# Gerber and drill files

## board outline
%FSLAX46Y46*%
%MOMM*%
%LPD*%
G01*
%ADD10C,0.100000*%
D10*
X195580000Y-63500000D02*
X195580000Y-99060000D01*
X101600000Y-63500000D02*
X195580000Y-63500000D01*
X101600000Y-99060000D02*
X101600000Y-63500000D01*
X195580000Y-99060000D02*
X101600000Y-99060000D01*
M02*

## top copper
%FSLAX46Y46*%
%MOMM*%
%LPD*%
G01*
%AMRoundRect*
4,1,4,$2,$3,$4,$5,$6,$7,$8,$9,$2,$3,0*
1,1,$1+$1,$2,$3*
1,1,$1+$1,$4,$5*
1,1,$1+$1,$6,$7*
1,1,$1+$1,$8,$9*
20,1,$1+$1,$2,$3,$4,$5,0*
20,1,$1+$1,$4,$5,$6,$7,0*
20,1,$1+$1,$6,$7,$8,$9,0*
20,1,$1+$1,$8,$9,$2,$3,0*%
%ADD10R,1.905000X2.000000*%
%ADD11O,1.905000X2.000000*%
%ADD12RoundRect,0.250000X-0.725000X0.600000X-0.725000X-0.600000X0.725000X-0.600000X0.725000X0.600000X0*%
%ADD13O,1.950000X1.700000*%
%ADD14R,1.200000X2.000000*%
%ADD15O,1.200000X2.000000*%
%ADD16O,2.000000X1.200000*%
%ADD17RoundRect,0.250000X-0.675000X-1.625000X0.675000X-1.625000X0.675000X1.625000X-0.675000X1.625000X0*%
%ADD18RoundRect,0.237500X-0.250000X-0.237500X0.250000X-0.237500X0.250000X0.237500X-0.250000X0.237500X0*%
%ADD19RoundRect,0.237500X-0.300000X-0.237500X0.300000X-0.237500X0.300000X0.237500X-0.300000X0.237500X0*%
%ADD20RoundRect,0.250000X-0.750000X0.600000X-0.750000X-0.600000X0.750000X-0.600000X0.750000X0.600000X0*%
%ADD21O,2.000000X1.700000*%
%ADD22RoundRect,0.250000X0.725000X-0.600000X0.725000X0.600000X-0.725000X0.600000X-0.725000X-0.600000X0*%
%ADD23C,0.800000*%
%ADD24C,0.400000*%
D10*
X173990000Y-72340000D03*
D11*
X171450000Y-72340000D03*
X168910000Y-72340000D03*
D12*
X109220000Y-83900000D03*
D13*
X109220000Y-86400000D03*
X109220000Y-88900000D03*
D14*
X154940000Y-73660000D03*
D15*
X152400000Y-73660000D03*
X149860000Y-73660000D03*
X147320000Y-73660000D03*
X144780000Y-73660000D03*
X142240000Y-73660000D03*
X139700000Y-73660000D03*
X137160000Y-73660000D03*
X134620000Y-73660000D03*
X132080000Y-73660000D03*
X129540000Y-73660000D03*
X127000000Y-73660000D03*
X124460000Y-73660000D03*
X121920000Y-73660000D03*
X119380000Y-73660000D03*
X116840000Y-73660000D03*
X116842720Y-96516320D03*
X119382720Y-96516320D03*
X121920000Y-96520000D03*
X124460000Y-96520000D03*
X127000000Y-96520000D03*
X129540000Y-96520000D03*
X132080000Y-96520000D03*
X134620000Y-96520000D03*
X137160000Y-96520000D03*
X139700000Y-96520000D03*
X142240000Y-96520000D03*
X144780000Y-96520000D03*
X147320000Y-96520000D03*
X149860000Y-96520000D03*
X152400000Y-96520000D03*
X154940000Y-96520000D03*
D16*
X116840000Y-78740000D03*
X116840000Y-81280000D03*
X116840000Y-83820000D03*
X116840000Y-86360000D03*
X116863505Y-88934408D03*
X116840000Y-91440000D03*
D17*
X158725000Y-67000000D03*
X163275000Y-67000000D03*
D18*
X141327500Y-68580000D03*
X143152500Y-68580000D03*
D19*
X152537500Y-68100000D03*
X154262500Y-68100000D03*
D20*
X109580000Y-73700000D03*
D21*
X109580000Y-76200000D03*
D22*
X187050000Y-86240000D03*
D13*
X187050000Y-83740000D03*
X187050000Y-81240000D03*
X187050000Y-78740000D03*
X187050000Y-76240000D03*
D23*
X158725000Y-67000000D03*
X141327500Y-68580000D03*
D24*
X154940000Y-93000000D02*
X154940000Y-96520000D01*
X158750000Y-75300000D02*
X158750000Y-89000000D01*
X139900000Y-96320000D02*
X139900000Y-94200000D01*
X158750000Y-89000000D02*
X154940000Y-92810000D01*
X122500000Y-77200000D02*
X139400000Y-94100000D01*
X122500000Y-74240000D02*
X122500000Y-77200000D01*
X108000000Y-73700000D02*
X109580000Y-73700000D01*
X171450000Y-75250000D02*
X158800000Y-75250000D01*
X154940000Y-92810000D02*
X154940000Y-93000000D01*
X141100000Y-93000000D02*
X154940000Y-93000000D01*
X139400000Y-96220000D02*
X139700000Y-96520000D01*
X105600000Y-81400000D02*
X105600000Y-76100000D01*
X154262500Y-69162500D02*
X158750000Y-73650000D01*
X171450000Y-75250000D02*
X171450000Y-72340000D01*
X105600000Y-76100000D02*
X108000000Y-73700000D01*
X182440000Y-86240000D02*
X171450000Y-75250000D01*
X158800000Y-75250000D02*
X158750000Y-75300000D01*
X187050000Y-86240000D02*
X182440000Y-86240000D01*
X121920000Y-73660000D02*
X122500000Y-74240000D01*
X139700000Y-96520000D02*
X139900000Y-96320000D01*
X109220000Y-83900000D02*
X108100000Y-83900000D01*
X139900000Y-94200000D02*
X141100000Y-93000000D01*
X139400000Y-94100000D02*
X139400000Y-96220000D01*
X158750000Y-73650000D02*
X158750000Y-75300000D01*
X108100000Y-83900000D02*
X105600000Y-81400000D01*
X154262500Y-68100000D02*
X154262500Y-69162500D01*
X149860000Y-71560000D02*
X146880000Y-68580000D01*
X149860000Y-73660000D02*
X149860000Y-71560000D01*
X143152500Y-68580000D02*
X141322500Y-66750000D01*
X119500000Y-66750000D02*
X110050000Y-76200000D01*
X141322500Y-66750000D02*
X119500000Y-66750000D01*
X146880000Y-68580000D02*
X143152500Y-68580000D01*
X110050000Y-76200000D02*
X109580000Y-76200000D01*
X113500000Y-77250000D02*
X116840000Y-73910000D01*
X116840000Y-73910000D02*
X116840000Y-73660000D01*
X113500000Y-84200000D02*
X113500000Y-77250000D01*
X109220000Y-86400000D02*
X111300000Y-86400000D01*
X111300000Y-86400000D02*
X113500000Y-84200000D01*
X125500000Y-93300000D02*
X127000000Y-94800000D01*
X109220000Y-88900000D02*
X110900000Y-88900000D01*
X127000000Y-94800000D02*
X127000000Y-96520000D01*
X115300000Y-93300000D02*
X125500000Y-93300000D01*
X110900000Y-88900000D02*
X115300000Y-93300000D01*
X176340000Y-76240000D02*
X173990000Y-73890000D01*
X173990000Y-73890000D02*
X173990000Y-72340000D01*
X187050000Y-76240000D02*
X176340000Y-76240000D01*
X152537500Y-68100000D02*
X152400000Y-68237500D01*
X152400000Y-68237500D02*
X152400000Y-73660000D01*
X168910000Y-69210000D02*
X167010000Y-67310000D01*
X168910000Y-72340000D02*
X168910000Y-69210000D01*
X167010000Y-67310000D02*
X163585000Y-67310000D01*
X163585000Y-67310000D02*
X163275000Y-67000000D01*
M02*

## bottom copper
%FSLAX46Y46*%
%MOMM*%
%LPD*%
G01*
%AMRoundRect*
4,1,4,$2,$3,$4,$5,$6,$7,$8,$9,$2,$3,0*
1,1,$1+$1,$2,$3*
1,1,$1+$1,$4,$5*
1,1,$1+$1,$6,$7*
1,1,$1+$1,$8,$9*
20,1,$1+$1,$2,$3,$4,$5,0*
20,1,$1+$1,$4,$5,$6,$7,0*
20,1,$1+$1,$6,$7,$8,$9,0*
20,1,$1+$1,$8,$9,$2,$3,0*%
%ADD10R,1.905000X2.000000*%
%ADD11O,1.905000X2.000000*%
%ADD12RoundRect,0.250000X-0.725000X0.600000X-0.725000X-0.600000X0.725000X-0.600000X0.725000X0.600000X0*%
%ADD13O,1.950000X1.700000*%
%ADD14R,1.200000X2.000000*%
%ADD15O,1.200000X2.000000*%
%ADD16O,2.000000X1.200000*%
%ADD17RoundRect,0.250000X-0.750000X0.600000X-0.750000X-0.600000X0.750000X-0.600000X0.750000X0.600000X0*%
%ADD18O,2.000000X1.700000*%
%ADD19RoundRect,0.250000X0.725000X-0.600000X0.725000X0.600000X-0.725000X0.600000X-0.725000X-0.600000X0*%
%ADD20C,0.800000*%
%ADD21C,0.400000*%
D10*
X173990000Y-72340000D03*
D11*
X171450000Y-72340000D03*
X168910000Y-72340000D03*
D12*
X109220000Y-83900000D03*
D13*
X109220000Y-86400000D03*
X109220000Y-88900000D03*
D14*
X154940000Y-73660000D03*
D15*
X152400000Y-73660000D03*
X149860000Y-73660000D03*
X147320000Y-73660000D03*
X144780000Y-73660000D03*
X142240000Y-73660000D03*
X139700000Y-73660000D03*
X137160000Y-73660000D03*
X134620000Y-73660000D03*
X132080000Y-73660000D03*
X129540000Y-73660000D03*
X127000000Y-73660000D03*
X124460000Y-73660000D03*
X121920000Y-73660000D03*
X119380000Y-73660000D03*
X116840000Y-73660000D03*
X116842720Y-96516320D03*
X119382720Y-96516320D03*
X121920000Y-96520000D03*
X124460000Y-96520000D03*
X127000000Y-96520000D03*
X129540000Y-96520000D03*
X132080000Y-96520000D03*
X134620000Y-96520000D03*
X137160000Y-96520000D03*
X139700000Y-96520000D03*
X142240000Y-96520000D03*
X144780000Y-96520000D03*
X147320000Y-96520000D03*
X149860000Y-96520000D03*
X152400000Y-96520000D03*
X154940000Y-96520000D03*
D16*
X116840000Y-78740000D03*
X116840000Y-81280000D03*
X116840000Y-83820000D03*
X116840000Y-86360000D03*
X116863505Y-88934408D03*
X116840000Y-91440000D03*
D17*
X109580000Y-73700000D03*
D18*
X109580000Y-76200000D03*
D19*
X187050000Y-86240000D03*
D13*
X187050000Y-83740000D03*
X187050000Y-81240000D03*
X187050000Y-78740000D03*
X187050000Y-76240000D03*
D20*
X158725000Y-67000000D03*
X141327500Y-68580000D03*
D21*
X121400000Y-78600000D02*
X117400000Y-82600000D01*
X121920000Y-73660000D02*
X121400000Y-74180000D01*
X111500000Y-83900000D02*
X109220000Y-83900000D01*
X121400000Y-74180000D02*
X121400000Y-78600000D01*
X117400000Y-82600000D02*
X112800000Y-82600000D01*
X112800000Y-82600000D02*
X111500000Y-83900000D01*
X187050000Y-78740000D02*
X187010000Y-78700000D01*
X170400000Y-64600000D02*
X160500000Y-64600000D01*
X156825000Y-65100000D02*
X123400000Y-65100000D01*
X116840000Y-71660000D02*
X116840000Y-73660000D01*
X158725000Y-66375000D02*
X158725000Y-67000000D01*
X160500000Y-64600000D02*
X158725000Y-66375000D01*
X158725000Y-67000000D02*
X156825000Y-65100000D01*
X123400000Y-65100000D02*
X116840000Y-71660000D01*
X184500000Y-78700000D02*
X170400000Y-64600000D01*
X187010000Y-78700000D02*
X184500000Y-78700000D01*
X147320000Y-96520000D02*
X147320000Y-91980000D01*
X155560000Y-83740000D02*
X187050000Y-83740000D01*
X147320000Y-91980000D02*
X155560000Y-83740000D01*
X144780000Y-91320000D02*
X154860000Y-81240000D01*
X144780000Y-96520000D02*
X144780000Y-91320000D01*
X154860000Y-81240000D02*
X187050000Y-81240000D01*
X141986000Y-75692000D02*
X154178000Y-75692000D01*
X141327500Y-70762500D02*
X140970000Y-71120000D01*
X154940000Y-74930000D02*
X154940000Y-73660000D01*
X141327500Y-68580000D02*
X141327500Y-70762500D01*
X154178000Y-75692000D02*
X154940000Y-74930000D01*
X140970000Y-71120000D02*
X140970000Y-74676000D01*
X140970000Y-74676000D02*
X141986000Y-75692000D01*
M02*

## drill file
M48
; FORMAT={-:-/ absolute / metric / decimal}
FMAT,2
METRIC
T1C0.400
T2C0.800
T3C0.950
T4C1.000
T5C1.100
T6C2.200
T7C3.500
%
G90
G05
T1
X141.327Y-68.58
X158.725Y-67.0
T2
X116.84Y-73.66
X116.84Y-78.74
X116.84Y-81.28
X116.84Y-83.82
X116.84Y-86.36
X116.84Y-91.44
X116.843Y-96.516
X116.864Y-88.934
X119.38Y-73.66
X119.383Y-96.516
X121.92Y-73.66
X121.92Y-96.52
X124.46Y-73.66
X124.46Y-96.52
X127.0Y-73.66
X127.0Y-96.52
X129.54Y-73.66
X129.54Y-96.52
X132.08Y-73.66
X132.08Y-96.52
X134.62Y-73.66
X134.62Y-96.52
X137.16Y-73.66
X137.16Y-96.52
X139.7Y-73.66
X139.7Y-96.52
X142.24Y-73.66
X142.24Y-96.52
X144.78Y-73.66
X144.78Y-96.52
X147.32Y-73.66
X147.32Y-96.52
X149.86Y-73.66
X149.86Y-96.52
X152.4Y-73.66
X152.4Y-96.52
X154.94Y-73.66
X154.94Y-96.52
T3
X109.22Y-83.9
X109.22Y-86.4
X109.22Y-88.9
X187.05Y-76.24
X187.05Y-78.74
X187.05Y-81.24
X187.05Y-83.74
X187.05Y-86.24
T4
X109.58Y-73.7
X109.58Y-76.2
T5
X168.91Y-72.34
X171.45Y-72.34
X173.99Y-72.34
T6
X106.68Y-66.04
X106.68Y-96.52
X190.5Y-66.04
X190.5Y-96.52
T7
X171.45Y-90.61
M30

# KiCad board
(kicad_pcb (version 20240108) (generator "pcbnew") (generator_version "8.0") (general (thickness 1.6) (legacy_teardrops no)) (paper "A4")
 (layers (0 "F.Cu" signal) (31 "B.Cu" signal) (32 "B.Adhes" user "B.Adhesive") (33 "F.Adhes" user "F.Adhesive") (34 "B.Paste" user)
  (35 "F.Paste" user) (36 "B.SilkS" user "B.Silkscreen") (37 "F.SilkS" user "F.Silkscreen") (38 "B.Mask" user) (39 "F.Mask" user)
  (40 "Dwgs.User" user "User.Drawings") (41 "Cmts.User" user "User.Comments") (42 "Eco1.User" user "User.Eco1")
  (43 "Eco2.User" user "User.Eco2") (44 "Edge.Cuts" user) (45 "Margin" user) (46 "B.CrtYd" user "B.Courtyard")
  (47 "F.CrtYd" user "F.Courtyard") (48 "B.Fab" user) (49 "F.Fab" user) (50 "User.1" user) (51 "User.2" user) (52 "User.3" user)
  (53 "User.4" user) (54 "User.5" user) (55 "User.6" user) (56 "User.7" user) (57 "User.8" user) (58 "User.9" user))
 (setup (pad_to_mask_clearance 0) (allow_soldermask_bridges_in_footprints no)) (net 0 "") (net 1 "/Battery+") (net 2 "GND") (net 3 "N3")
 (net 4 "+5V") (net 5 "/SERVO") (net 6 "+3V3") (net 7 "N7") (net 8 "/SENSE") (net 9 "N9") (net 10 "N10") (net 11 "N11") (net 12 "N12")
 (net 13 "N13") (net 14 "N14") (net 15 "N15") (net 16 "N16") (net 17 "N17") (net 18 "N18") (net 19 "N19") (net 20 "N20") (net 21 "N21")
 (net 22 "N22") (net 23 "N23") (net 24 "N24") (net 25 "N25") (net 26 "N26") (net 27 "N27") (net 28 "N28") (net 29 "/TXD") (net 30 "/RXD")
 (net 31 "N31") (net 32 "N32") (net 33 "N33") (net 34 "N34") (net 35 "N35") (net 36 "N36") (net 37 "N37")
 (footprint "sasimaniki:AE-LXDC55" (layer "F.Cu") (at 173.99 72.34 180)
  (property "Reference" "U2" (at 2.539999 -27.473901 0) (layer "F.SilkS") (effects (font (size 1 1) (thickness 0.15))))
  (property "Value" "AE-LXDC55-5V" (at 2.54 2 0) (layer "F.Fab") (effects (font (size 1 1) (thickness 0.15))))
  (pad "" np_thru_hole oval (at 2.54 -18.27 180) (size 3.5 3.5) (drill 3.5) (layers "F&B.Cu" "*.Mask"))
  (pad "1" thru_hole rect (at 0 0 180) (size 1.905 2) (drill 1.1) (layers "*.Cu" "*.Mask") (remove_unused_layers no) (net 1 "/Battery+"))
  (pad "2" thru_hole oval (at 2.54 0 180) (size 1.905 2) (drill 1.1) (layers "*.Cu" "*.Mask") (remove_unused_layers no) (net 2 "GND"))
  (pad "3" thru_hole oval (at 5.08 0 180) (size 1.905 2) (drill 1.1) (layers "*.Cu" "*.Mask") (remove_unused_layers no) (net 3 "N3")))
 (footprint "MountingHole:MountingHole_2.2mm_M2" (layer "F.Cu") (at 106.68 96.52)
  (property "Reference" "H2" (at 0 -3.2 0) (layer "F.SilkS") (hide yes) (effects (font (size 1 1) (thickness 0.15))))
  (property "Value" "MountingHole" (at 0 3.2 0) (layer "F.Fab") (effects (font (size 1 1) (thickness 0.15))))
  (pad "" np_thru_hole circle (at 0 0) (size 2.2 2.2) (drill 2.2) (layers "*.Cu" "*.Mask")))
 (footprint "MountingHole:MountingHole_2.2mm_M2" (layer "F.Cu") (at 190.5 66.04)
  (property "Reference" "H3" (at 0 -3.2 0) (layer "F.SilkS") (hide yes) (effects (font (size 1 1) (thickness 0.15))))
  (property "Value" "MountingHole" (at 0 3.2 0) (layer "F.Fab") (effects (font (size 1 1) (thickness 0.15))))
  (pad "" np_thru_hole circle (at 0 0) (size 2.2 2.2) (drill 2.2) (layers "*.Cu" "*.Mask")))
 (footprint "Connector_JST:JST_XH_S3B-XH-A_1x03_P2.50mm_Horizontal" (layer "F.Cu") (at 109.22 83.9 -90)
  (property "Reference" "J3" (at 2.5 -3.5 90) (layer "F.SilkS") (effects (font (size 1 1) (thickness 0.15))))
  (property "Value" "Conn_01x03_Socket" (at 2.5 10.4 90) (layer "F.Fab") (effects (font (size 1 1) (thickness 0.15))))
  (pad "1" thru_hole roundrect (at 0 0 270) (size 1.7 1.95) (drill 0.95) (layers "*.Cu" "*.Mask") (remove_unused_layers no)
   (roundrect_rratio 0.147059) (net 2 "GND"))
  (pad "2" thru_hole oval (at 2.5 0 270) (size 1.7 1.95) (drill 0.95) (layers "*.Cu" "*.Mask") (remove_unused_layers no) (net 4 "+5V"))
  (pad "3" thru_hole oval (at 5 0 270) (size 1.7 1.95) (drill 0.95) (layers "*.Cu" "*.Mask") (remove_unused_layers no) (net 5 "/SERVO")))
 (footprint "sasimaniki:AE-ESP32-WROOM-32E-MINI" (layer "F.Cu") (at 154.94 73.66 -90)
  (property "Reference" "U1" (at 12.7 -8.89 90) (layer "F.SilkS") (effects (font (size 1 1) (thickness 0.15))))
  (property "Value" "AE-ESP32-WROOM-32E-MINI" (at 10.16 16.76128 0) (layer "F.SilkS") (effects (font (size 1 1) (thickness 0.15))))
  (pad "1" thru_hole rect (at 0 0 180) (size 1.2 2) (drill 0.8) (layers "*.Cu" "*.Mask") (remove_unused_layers no) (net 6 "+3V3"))
  (pad "2" thru_hole oval (at 0 2.54 180) (size 1.2 2) (drill 0.8) (layers "*.Cu" "*.Mask") (remove_unused_layers no) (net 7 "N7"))
  (pad "3" thru_hole oval (at 0 5.08 180) (size 1.2 2) (drill 0.8) (layers "*.Cu" "*.Mask") (remove_unused_layers no) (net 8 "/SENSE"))
  (pad "4" thru_hole oval (at 0 7.62 180) (size 1.2 2) (drill 0.8) (layers "*.Cu" "*.Mask") (remove_unused_layers no) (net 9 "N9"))
  (pad "5" thru_hole oval (at 0 10.16 180) (size 1.2 2) (drill 0.8) (layers "*.Cu" "*.Mask") (remove_unused_layers no) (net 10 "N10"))
  (pad "6" thru_hole oval (at 0 12.7 180) (size 1.2 2) (drill 0.8) (layers "*.Cu" "*.Mask") (remove_unused_layers no) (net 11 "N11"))
  (pad "7" thru_hole oval (at 0 15.24 180) (size 1.2 2) (drill 0.8) (layers "*.Cu" "*.Mask") (remove_unused_layers no) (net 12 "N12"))
  (pad "8" thru_hole oval (at 0 17.78 180) (size 1.2 2) (drill 0.8) (layers "*.Cu" "*.Mask") (remove_unused_layers no) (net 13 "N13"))
  (pad "9" thru_hole oval (at 0 20.32 180) (size 1.2 2) (drill 0.8) (layers "*.Cu" "*.Mask") (remove_unused_layers no) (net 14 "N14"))
  (pad "10" thru_hole oval (at 0 22.86 180) (size 1.2 2) (drill 0.8) (layers "*.Cu" "*.Mask") (remove_unused_layers no) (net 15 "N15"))
  (pad "11" thru_hole oval (at 0 25.4 180) (size 1.2 2) (drill 0.8) (layers "*.Cu" "*.Mask") (remove_unused_layers no) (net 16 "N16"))
  (pad "12" thru_hole oval (at 0 27.94 180) (size 1.2 2) (drill 0.8) (layers "*.Cu" "*.Mask") (remove_unused_layers no) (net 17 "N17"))
  (pad "13" thru_hole oval (at 0 30.48 180) (size 1.2 2) (drill 0.8) (layers "*.Cu" "*.Mask") (remove_unused_layers no) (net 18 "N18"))
  (pad "14" thru_hole oval (at 0 33.02 180) (size 1.2 2) (drill 0.8) (layers "*.Cu" "*.Mask") (remove_unused_layers no) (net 2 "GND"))
  (pad "15" thru_hole oval (at 0 35.56 180) (size 1.2 2) (drill 0.8) (layers "*.Cu" "*.Mask") (remove_unused_layers no) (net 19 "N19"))
  (pad "16" thru_hole oval (at 0 38.1 180) (size 1.2 2) (drill 0.8) (layers "*.Cu" "*.Mask") (remove_unused_layers no) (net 4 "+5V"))
  (pad "17" thru_hole oval (at 22.85632 38.09728 180) (size 1.2 2) (drill 0.8) (layers "*.Cu" "*.Mask") (remove_unused_layers no)
   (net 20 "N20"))
  (pad "18" thru_hole oval (at 22.85632 35.55728 180) (size 1.2 2) (drill 0.8) (layers "*.Cu" "*.Mask") (remove_unused_layers no)
   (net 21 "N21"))
  (pad "19" thru_hole oval (at 22.86 33.02 180) (size 1.2 2) (drill 0.8) (layers "*.Cu" "*.Mask") (remove_unused_layers no) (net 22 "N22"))
  (pad "20" thru_hole oval (at 22.86 30.48 180) (size 1.2 2) (drill 0.8) (layers "*.Cu" "*.Mask") (remove_unused_layers no) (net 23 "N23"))
  (pad "21" thru_hole oval (at 22.86 27.94 180) (size 1.2 2) (drill 0.8) (layers "*.Cu" "*.Mask") (remove_unused_layers no) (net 5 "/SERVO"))
  (pad "22" thru_hole oval (at 22.86 25.4 180) (size 1.2 2) (drill 0.8) (layers "*.Cu" "*.Mask") (remove_unused_layers no) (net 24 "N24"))
  (pad "23" thru_hole oval (at 22.86 22.86 180) (size 1.2 2) (drill 0.8) (layers "*.Cu" "*.Mask") (remove_unused_layers no) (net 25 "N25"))
  (pad "24" thru_hole oval (at 22.86 20.32 180) (size 1.2 2) (drill 0.8) (layers "*.Cu" "*.Mask") (remove_unused_layers no) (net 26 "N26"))
  (pad "25" thru_hole oval (at 22.86 17.78 180) (size 1.2 2) (drill 0.8) (layers "*.Cu" "*.Mask") (remove_unused_layers no) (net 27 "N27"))
  (pad "26" thru_hole oval (at 22.86 15.24 180) (size 1.2 2) (drill 0.8) (layers "*.Cu" "*.Mask") (remove_unused_layers no) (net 2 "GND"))
  (pad "27" thru_hole oval (at 22.86 12.7 180) (size 1.2 2) (drill 0.8) (layers "*.Cu" "*.Mask") (remove_unused_layers no) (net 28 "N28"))
  (pad "28" thru_hole oval (at 22.86 10.16 180) (size 1.2 2) (drill 0.8) (layers "*.Cu" "*.Mask") (remove_unused_layers no) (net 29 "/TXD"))
  (pad "29" thru_hole oval (at 22.86 7.62 180) (size 1.2 2) (drill 0.8) (layers "*.Cu" "*.Mask") (remove_unused_layers no) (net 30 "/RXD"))
  (pad "30" thru_hole oval (at 22.86 5.08 180) (size 1.2 2) (drill 0.8) (layers "*.Cu" "*.Mask") (remove_unused_layers no) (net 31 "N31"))
  (pad "31" thru_hole oval (at 22.86 2.54 180) (size 1.2 2) (drill 0.8) (layers "*.Cu" "*.Mask") (remove_unused_layers no) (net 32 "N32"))
  (pad "32" thru_hole oval (at 22.86 0 180) (size 1.2 2) (drill 0.8) (layers "*.Cu" "*.Mask") (remove_unused_layers no) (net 2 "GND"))
  (pad "33" thru_hole oval (at 5.08 38.1 180) (size 2 1.2) (drill 0.8) (layers "*.Cu" "*.Mask") (remove_unused_layers no))
  (pad "34" thru_hole oval (at 7.62 38.1 180) (size 2 1.2) (drill 0.8) (layers "*.Cu" "*.Mask") (remove_unused_layers no) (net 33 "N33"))
  (pad "35" thru_hole oval (at 10.16 38.1 180) (size 2 1.2) (drill 0.8) (layers "*.Cu" "*.Mask") (remove_unused_layers no) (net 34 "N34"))
  (pad "36" thru_hole oval (at 12.7 38.1 180) (size 2 1.2) (drill 0.8) (layers "*.Cu" "*.Mask") (remove_unused_layers no) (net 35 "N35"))
  (pad "37" thru_hole oval (at 15.274408 38.076495 180) (size 2 1.2) (drill 0.8) (layers "*.Cu" "*.Mask") (remove_unused_layers no)
   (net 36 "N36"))
  (pad "38" thru_hole oval (at 17.78 38.1 180) (size 2 1.2) (drill 0.8) (layers "*.Cu" "*.Mask") (remove_unused_layers no) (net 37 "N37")))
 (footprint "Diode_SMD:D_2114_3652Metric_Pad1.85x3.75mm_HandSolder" (layer "F.Cu") (at 161 67)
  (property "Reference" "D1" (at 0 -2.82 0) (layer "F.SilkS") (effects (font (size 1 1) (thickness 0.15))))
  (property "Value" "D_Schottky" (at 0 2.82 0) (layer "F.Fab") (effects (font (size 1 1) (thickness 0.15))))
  (pad "1" smd roundrect (at -2.275 0) (size 1.85 3.75) (layers "F.Cu" "F.Paste" "F.Mask") (roundrect_rratio 0.135135) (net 4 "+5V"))
  (pad "2" smd roundrect (at 2.275 0) (size 1.85 3.75) (layers "F.Cu" "F.Paste" "F.Mask") (roundrect_rratio 0.135135) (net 3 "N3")))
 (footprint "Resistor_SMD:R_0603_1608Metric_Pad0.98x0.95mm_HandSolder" (layer "F.Cu") (at 142.24 68.58)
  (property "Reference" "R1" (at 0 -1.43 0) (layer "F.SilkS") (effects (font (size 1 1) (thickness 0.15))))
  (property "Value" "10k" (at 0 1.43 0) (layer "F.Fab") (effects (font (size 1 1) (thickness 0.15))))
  (pad "1" smd roundrect (at -0.9125 0) (size 0.975 0.95) (layers "F.Cu" "F.Paste" "F.Mask") (roundrect_rratio 0.25) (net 6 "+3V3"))
  (pad "2" smd roundrect (at 0.9125 0) (size 0.975 0.95) (layers "F.Cu" "F.Paste" "F.Mask") (roundrect_rratio 0.25) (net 8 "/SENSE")))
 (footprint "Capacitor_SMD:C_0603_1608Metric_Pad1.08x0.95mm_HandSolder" (layer "F.Cu") (at 153.4 68.1)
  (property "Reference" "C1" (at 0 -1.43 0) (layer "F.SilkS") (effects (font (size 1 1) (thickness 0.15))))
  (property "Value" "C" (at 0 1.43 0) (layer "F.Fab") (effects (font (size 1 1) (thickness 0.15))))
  (pad "1" smd roundrect (at -0.8625 0) (size 1.075 0.95) (layers "F.Cu" "F.Paste" "F.Mask") (roundrect_rratio 0.25) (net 7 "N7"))
  (pad "2" smd roundrect (at 0.8625 0) (size 1.075 0.95) (layers "F.Cu" "F.Paste" "F.Mask") (roundrect_rratio 0.25) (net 2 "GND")))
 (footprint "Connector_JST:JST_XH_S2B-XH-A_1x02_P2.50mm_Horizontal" (layer "F.Cu") (at 109.58 73.7 -90)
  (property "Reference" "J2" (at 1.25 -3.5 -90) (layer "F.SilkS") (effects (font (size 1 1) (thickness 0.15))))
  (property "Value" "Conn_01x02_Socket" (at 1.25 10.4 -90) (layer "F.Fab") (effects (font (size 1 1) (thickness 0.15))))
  (pad "1" thru_hole roundrect (at 0 0 270) (size 1.7 2) (drill 1) (layers "*.Cu" "*.Mask") (remove_unused_layers no)
   (roundrect_rratio 0.147059) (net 2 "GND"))
  (pad "2" thru_hole oval (at 2.5 0 270) (size 1.7 2) (drill 1) (layers "*.Cu" "*.Mask") (remove_unused_layers no) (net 8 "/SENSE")))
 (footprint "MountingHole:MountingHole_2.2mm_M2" (layer "F.Cu") (at 106.68 66.04)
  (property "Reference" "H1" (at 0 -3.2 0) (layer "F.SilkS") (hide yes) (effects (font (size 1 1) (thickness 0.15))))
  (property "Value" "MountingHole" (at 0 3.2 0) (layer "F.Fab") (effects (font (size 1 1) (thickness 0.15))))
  (pad "" np_thru_hole circle (at 0 0) (size 2.2 2.2) (drill 2.2) (layers "*.Cu" "*.Mask")))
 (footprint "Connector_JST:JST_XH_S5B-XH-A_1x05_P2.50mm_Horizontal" (layer "F.Cu") (at 187.05 86.24 90)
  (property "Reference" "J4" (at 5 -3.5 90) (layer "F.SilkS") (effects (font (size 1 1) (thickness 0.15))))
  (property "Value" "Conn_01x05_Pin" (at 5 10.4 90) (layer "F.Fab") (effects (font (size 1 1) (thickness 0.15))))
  (pad "1" thru_hole roundrect (at 0 0 90) (size 1.7 1.95) (drill 0.95) (layers "*.Cu" "*.Mask") (remove_unused_layers no)
   (roundrect_rratio 0.147059) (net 2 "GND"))
  (pad "2" thru_hole oval (at 2.5 0 90) (size 1.7 1.95) (drill 0.95) (layers "*.Cu" "*.Mask") (remove_unused_layers no) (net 30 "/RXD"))
  (pad "3" thru_hole oval (at 5 0 90) (size 1.7 1.95) (drill 0.95) (layers "*.Cu" "*.Mask") (remove_unused_layers no) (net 29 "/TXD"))
  (pad "4" thru_hole oval (at 7.5 0 90) (size 1.7 1.95) (drill 0.95) (layers "*.Cu" "*.Mask") (remove_unused_layers no) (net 4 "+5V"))
  (pad "5" thru_hole oval (at 10 0 90) (size 1.7 1.95) (drill 0.95) (layers "*.Cu" "*.Mask") (remove_unused_layers no) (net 1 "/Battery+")))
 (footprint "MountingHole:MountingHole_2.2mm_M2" (layer "F.Cu") (at 190.5 96.52)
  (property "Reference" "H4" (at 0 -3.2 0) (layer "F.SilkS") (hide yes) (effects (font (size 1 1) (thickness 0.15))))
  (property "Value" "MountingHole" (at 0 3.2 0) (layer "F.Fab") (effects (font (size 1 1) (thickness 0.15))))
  (pad "" np_thru_hole circle (at 0 0) (size 2.2 2.2) (drill 2.2) (layers "*.Cu" "*.Mask")))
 (gr_line (start 195.58 63.5) (end 195.58 99.06) (stroke (width 0.1) (type default)) (layer "Edge.Cuts"))
 (gr_line (start 101.6 63.5) (end 195.58 63.5) (stroke (width 0.1) (type default)) (layer "Edge.Cuts"))
 (gr_line (start 101.6 99.06) (end 101.6 63.5) (stroke (width 0.1) (type default)) (layer "Edge.Cuts"))
 (gr_line (start 195.58 99.06) (end 101.6 99.06) (stroke (width 0.1) (type default)) (layer "Edge.Cuts"))
 (segment (start 154.94 93) (end 154.94 96.52) (width 0.4) (layer "F.Cu") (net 2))
 (segment (start 158.75 75.3) (end 158.75 89) (width 0.4) (layer "F.Cu") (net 2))
 (segment (start 139.9 96.32) (end 139.9 94.2) (width 0.4) (layer "F.Cu") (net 2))
 (segment (start 158.75 89) (end 154.94 92.81) (width 0.4) (layer "F.Cu") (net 2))
 (segment (start 122.5 77.2) (end 139.4 94.1) (width 0.4) (layer "F.Cu") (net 2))
 (segment (start 122.5 74.24) (end 122.5 77.2) (width 0.4) (layer "F.Cu") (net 2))
 (segment (start 108 73.7) (end 109.58 73.7) (width 0.4) (layer "F.Cu") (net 2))
 (segment (start 171.45 75.25) (end 158.8 75.25) (width 0.4) (layer "F.Cu") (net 2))
 (segment (start 154.94 92.81) (end 154.94 93) (width 0.4) (layer "F.Cu") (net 2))
 (segment (start 141.1 93) (end 154.94 93) (width 0.4) (layer "F.Cu") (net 2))
 (segment (start 139.4 96.22) (end 139.7 96.52) (width 0.4) (layer "F.Cu") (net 2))
 (segment (start 105.6 81.4) (end 105.6 76.1) (width 0.4) (layer "F.Cu") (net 2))
 (segment (start 154.2625 69.1625) (end 158.75 73.65) (width 0.4) (layer "F.Cu") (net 2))
 (segment (start 171.45 75.25) (end 171.45 72.34) (width 0.4) (layer "F.Cu") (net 2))
 (segment (start 105.6 76.1) (end 108 73.7) (width 0.4) (layer "F.Cu") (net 2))
 (segment (start 182.44 86.24) (end 171.45 75.25) (width 0.4) (layer "F.Cu") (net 2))
 (segment (start 158.8 75.25) (end 158.75 75.3) (width 0.4) (layer "F.Cu") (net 2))
 (segment (start 187.05 86.24) (end 182.44 86.24) (width 0.4) (layer "F.Cu") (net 2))
 (segment (start 121.92 73.66) (end 122.5 74.24) (width 0.4) (layer "F.Cu") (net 2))
 (segment (start 139.7 96.52) (end 139.9 96.32) (width 0.4) (layer "F.Cu") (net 2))
 (segment (start 109.22 83.9) (end 108.1 83.9) (width 0.4) (layer "F.Cu") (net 2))
 (segment (start 139.9 94.2) (end 141.1 93) (width 0.4) (layer "F.Cu") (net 2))
 (segment (start 139.4 94.1) (end 139.4 96.22) (width 0.4) (layer "F.Cu") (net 2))
 (segment (start 158.75 73.65) (end 158.75 75.3) (width 0.4) (layer "F.Cu") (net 2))
 (segment (start 108.1 83.9) (end 105.6 81.4) (width 0.4) (layer "F.Cu") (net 2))
 (segment (start 154.2625 68.1) (end 154.2625 69.1625) (width 0.4) (layer "F.Cu") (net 2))
 (segment (start 121.4 78.6) (end 117.4 82.6) (width 0.4) (layer "B.Cu") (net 2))
 (segment (start 121.92 73.66) (end 121.4 74.18) (width 0.4) (layer "B.Cu") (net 2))
 (segment (start 111.5 83.9) (end 109.22 83.9) (width 0.4) (layer "B.Cu") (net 2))
 (segment (start 121.4 74.18) (end 121.4 78.6) (width 0.4) (layer "B.Cu") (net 2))
 (segment (start 117.4 82.6) (end 112.8 82.6) (width 0.4) (layer "B.Cu") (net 2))
 (segment (start 112.8 82.6) (end 111.5 83.9) (width 0.4) (layer "B.Cu") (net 2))
 (segment (start 149.86 71.56) (end 146.88 68.58) (width 0.4) (layer "F.Cu") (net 8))
 (segment (start 149.86 73.66) (end 149.86 71.56) (width 0.4) (layer "F.Cu") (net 8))
 (segment (start 143.1525 68.58) (end 141.3225 66.75) (width 0.4) (layer "F.Cu") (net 8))
 (segment (start 119.5 66.75) (end 110.05 76.2) (width 0.4) (layer "F.Cu") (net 8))
 (segment (start 141.3225 66.75) (end 119.5 66.75) (width 0.4) (layer "F.Cu") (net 8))
 (segment (start 146.88 68.58) (end 143.1525 68.58) (width 0.4) (layer "F.Cu") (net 8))
 (segment (start 110.05 76.2) (end 109.58 76.2) (width 0.4) (layer "F.Cu") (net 8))
 (segment (start 113.5 77.25) (end 116.84 73.91) (width 0.4) (layer "F.Cu") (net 4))
 (segment (start 116.84 73.91) (end 116.84 73.66) (width 0.4) (layer "F.Cu") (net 4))
 (segment (start 113.5 84.2) (end 113.5 77.25) (width 0.4) (layer "F.Cu") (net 4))
 (segment (start 109.22 86.4) (end 111.3 86.4) (width 0.4) (layer "F.Cu") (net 4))
 (segment (start 111.3 86.4) (end 113.5 84.2) (width 0.4) (layer "F.Cu") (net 4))
 (via (at 158.725 67) (size 0.8) (drill 0.4) (layers "F.Cu" "B.Cu") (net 4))
 (segment (start 187.05 78.74) (end 187.01 78.7) (width 0.4) (layer "B.Cu") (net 4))
 (segment (start 170.4 64.6) (end 160.5 64.6) (width 0.4) (layer "B.Cu") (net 4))
 (segment (start 156.825 65.1) (end 123.4 65.1) (width 0.4) (layer "B.Cu") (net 4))
 (segment (start 116.84 71.66) (end 116.84 73.66) (width 0.4) (layer "B.Cu") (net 4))
 (segment (start 158.725 66.375) (end 158.725 67) (width 0.4) (layer "B.Cu") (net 4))
 (segment (start 160.5 64.6) (end 158.725 66.375) (width 0.4) (layer "B.Cu") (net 4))
 (segment (start 158.725 67) (end 156.825 65.1) (width 0.4) (layer "B.Cu") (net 4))
 (segment (start 123.4 65.1) (end 116.84 71.66) (width 0.4) (layer "B.Cu") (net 4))
 (segment (start 184.5 78.7) (end 170.4 64.6) (width 0.4) (layer "B.Cu") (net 4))
 (segment (start 187.01 78.7) (end 184.5 78.7) (width 0.4) (layer "B.Cu") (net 4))
 (segment (start 125.5 93.3) (end 127 94.8) (width 0.4) (layer "F.Cu") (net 5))
 (segment (start 109.22 88.9) (end 110.9 88.9) (width 0.4) (layer "F.Cu") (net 5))
 (segment (start 127 94.8) (end 127 96.52) (width 0.4) (layer "F.Cu") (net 5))
 (segment (start 115.3 93.3) (end 125.5 93.3) (width 0.4) (layer "F.Cu") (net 5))
 (segment (start 110.9 88.9) (end 115.3 93.3) (width 0.4) (layer "F.Cu") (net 5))
 (segment (start 147.32 96.52) (end 147.32 91.98) (width 0.4) (layer "B.Cu") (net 30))
 (segment (start 155.56 83.74) (end 187.05 83.74) (width 0.4) (layer "B.Cu") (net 30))
 (segment (start 147.32 91.98) (end 155.56 83.74) (width 0.4) (layer "B.Cu") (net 30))
 (segment (start 144.78 91.32) (end 154.86 81.24) (width 0.4) (layer "B.Cu") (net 29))
 (segment (start 144.78 96.52) (end 144.78 91.32) (width 0.4) (layer "B.Cu") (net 29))
 (segment (start 154.86 81.24) (end 187.05 81.24) (width 0.4) (layer "B.Cu") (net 29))
 (segment (start 176.34 76.24) (end 173.99 73.89) (width 0.4) (layer "F.Cu") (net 1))
 (segment (start 173.99 73.89) (end 173.99 72.34) (width 0.4) (layer "F.Cu") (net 1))
 (segment (start 187.05 76.24) (end 176.34 76.24) (width 0.4) (layer "F.Cu") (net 1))
 (segment (start 152.5375 68.1) (end 152.4 68.2375) (width 0.4) (layer "F.Cu") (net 7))
 (segment (start 152.4 68.2375) (end 152.4 73.66) (width 0.4) (layer "F.Cu") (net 7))
 (segment (start 168.91 69.21) (end 167.01 67.31) (width 0.4) (layer "F.Cu") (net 3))
 (segment (start 168.91 72.34) (end 168.91 69.21) (width 0.4) (layer "F.Cu") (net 3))
 (segment (start 167.01 67.31) (end 163.585 67.31) (width 0.4) (layer "F.Cu") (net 3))
 (segment (start 163.585 67.31) (end 163.275 67) (width 0.4) (layer "F.Cu") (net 3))
 (via (at 141.3275 68.58) (size 0.8) (drill 0.4) (layers "F.Cu" "B.Cu") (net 6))
 (segment (start 141.986 75.692) (end 154.178 75.692) (width 0.4) (layer "B.Cu") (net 6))
 (segment (start 141.3275 70.7625) (end 140.97 71.12) (width 0.4) (layer "B.Cu") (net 6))
 (segment (start 154.94 74.93) (end 154.94 73.66) (width 0.4) (layer "B.Cu") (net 6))
 (segment (start 141.3275 68.58) (end 141.3275 70.7625) (width 0.4) (layer "B.Cu") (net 6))
 (segment (start 154.178 75.692) (end 154.94 74.93) (width 0.4) (layer "B.Cu") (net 6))
 (segment (start 140.97 71.12) (end 140.97 74.676) (width 0.4) (layer "B.Cu") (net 6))
 (segment (start 140.97 74.676) (end 141.986 75.692) (width 0.4) (layer "B.Cu") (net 6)))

